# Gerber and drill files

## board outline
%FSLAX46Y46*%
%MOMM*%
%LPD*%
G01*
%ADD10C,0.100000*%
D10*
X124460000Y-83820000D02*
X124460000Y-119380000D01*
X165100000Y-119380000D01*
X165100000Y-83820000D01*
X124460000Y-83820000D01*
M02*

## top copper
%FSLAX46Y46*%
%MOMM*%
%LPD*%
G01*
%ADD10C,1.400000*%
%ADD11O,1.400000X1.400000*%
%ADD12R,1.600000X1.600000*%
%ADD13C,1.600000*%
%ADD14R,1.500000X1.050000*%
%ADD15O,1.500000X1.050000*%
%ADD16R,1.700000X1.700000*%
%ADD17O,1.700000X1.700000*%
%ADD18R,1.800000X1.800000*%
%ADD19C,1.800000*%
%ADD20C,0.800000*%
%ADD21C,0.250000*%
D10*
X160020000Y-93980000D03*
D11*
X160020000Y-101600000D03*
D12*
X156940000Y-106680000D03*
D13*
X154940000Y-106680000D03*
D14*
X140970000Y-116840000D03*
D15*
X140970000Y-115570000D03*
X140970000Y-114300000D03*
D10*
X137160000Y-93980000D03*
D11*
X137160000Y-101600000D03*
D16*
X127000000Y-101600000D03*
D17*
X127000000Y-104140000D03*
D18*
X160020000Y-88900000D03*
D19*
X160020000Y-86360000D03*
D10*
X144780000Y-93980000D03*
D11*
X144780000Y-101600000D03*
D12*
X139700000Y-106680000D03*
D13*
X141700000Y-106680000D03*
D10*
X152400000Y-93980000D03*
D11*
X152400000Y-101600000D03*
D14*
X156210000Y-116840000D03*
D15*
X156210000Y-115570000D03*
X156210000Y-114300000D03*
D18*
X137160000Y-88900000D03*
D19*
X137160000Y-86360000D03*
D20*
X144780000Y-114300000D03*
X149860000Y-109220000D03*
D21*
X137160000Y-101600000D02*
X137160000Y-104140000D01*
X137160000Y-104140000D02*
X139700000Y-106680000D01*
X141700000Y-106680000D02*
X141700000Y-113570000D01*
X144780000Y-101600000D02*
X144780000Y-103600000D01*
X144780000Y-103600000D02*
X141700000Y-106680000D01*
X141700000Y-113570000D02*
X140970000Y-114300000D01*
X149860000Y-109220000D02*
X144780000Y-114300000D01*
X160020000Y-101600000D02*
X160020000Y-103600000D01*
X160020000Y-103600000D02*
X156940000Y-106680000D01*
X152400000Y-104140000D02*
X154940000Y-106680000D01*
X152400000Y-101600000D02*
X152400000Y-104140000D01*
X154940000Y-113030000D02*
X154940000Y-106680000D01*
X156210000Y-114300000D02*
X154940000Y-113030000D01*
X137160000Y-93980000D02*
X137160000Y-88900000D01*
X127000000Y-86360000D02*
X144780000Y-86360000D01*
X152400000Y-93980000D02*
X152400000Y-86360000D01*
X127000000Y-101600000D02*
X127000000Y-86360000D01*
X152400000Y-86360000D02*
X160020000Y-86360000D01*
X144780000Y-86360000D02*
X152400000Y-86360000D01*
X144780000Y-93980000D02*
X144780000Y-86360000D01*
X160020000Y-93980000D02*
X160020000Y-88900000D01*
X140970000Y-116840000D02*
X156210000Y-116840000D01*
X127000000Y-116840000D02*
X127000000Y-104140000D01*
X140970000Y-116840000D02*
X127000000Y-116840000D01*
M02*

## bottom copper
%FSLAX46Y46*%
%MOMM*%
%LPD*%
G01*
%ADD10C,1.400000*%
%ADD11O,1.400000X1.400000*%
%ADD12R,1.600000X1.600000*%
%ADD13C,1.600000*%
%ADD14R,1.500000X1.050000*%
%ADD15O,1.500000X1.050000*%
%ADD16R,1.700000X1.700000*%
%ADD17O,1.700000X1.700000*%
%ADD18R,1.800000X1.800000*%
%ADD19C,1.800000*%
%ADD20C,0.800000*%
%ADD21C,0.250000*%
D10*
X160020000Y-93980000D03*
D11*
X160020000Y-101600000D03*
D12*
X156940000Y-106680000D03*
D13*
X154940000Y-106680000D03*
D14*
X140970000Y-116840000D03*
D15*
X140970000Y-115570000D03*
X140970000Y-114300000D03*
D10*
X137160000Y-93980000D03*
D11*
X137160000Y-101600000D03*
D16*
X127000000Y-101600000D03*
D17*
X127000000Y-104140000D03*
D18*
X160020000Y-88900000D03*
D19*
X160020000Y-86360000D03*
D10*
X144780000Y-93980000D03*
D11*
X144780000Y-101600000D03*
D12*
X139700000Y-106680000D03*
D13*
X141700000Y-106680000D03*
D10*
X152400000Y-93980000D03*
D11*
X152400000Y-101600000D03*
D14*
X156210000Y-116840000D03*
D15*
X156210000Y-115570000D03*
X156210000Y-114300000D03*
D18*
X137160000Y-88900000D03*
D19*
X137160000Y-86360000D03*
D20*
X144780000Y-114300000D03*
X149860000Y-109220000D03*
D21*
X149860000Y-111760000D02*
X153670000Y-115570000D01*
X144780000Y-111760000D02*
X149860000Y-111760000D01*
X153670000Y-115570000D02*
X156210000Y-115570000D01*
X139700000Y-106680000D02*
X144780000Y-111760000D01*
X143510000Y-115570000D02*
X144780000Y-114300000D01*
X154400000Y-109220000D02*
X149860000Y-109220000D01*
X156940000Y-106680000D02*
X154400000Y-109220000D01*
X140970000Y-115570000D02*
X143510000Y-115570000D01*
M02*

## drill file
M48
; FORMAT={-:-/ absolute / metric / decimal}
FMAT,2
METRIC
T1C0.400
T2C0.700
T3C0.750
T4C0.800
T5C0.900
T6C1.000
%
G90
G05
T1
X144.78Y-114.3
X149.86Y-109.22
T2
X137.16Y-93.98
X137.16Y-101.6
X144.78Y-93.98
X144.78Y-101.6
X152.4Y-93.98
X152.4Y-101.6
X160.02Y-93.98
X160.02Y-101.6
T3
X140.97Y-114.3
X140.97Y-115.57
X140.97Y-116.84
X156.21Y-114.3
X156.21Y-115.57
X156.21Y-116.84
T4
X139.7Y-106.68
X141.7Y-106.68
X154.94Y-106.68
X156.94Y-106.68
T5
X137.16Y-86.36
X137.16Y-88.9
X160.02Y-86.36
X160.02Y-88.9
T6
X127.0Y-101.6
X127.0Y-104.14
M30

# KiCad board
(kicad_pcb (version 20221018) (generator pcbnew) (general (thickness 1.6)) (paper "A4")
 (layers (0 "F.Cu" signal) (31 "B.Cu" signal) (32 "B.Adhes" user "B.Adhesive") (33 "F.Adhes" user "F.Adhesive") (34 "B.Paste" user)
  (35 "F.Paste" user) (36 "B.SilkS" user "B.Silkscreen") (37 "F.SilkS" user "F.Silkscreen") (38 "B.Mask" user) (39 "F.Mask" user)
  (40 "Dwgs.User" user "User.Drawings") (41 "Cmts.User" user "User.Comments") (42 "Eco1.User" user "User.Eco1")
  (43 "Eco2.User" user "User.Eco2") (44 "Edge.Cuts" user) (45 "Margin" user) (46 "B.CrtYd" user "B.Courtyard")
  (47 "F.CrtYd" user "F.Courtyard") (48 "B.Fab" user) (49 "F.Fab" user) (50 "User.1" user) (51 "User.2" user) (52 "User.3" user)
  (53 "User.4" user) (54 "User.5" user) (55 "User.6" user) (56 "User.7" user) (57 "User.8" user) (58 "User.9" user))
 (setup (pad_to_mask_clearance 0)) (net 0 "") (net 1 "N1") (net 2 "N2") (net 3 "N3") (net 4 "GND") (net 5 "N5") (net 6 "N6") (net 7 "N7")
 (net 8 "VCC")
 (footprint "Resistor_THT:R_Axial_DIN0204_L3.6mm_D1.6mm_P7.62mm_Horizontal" (layer "F.Cu") (at 160.02 93.98 -90)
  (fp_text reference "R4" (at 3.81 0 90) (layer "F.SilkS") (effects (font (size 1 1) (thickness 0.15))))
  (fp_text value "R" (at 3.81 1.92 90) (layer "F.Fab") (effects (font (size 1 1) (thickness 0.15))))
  (pad "1" thru_hole circle (at 0 0 270) (size 1.4 1.4) (drill 0.7) (layers "*.Cu" "*.Mask") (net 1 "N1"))
  (pad "2" thru_hole oval (at 7.62 0 270) (size 1.4 1.4) (drill 0.7) (layers "*.Cu" "*.Mask") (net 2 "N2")))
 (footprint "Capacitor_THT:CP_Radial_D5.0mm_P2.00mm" (layer "F.Cu") (at 156.94 106.68 180)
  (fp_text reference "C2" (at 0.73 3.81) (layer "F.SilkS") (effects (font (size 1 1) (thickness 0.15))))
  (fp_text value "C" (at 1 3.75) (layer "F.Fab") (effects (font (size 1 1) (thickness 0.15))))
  (pad "1" thru_hole rect (at 0 0 180) (size 1.6 1.6) (drill 0.8) (layers "*.Cu" "*.Mask") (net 2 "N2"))
  (pad "2" thru_hole circle (at 2 0 180) (size 1.6 1.6) (drill 0.8) (layers "*.Cu" "*.Mask") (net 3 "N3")))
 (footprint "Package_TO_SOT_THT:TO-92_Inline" (layer "F.Cu") (at 140.97 116.84 90)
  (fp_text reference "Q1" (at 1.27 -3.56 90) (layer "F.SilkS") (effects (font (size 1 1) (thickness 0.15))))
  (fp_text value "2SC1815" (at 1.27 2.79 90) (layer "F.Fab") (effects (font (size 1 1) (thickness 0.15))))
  (pad "1" thru_hole rect (at 0 0 90) (size 1.05 1.5) (drill 0.75) (layers "*.Cu" "*.Mask") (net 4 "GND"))
  (pad "2" thru_hole oval (at 1.27 0 90) (size 1.05 1.5) (drill 0.75) (layers "*.Cu" "*.Mask") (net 2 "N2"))
  (pad "3" thru_hole oval (at 2.54 0 90) (size 1.05 1.5) (drill 0.75) (layers "*.Cu" "*.Mask") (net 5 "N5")))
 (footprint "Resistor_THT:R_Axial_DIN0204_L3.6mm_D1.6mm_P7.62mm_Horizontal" (layer "F.Cu") (at 137.16 93.98 -90)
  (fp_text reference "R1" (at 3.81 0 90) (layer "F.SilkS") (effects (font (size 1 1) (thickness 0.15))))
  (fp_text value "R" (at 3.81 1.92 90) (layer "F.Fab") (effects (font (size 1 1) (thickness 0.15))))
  (pad "1" thru_hole circle (at 0 0 270) (size 1.4 1.4) (drill 0.7) (layers "*.Cu" "*.Mask") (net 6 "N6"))
  (pad "2" thru_hole oval (at 7.62 0 270) (size 1.4 1.4) (drill 0.7) (layers "*.Cu" "*.Mask") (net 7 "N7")))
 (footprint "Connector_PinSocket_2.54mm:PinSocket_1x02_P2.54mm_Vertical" (layer "F.Cu") (at 127 101.6)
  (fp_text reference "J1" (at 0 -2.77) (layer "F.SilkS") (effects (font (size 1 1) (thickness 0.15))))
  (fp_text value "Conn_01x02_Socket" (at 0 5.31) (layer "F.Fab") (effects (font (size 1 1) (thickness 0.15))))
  (pad "1" thru_hole rect (at 0 0) (size 1.7 1.7) (drill 1) (layers "*.Cu" "*.Mask") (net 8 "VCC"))
  (pad "2" thru_hole oval (at 0 2.54) (size 1.7 1.7) (drill 1) (layers "*.Cu" "*.Mask") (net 4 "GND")))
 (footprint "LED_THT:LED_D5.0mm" (layer "F.Cu") (at 160.02 88.9 90)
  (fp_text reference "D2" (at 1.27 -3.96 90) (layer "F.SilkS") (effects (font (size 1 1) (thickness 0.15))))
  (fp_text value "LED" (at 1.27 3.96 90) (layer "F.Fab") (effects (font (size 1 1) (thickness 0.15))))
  (pad "1" thru_hole rect (at 0 0 90) (size 1.8 1.8) (drill 0.9) (layers "*.Cu" "*.Mask") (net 1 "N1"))
  (pad "2" thru_hole circle (at 2.54 0 90) (size 1.8 1.8) (drill 0.9) (layers "*.Cu" "*.Mask") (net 8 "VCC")))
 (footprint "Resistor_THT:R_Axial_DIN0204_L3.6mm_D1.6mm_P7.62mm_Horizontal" (layer "F.Cu") (at 144.78 93.98 -90)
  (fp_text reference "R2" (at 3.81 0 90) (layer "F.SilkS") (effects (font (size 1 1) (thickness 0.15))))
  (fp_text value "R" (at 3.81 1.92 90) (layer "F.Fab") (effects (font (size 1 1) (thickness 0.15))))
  (pad "1" thru_hole circle (at 0 0 270) (size 1.4 1.4) (drill 0.7) (layers "*.Cu" "*.Mask") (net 8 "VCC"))
  (pad "2" thru_hole oval (at 7.62 0 270) (size 1.4 1.4) (drill 0.7) (layers "*.Cu" "*.Mask") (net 5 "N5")))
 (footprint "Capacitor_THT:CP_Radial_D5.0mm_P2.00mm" (layer "F.Cu") (at 139.7 106.68)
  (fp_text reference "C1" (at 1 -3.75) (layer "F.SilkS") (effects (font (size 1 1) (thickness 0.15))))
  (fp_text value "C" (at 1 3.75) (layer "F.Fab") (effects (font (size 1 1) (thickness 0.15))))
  (pad "1" thru_hole rect (at 0 0) (size 1.6 1.6) (drill 0.8) (layers "*.Cu" "*.Mask") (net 7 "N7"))
  (pad "2" thru_hole circle (at 2 0) (size 1.6 1.6) (drill 0.8) (layers "*.Cu" "*.Mask") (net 5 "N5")))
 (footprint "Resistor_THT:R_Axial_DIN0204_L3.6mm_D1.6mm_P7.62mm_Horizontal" (layer "F.Cu") (at 152.4 93.98 -90)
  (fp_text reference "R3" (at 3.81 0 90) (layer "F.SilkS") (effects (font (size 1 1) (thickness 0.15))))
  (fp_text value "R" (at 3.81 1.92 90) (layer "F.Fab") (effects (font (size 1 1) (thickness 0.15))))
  (pad "1" thru_hole circle (at 0 0 270) (size 1.4 1.4) (drill 0.7) (layers "*.Cu" "*.Mask") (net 8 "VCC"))
  (pad "2" thru_hole oval (at 7.62 0 270) (size 1.4 1.4) (drill 0.7) (layers "*.Cu" "*.Mask") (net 3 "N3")))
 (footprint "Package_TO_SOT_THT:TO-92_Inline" (layer "F.Cu") (at 156.21 116.84 90)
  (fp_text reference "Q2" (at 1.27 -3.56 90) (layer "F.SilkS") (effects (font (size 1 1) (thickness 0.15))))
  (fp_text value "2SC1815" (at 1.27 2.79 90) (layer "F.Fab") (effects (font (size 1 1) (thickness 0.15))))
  (pad "1" thru_hole rect (at 0 0 90) (size 1.05 1.5) (drill 0.75) (layers "*.Cu" "*.Mask") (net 4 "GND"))
  (pad "2" thru_hole oval (at 1.27 0 90) (size 1.05 1.5) (drill 0.75) (layers "*.Cu" "*.Mask") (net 7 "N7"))
  (pad "3" thru_hole oval (at 2.54 0 90) (size 1.05 1.5) (drill 0.75) (layers "*.Cu" "*.Mask") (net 3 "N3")))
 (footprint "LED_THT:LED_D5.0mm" (layer "F.Cu") (at 137.16 88.9 90)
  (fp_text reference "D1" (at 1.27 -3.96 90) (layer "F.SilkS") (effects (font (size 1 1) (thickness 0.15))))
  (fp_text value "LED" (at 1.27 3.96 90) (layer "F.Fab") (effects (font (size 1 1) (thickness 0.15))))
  (pad "1" thru_hole rect (at 0 0 90) (size 1.8 1.8) (drill 0.9) (layers "*.Cu" "*.Mask") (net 6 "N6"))
  (pad "2" thru_hole circle (at 2.54 0 90) (size 1.8 1.8) (drill 0.9) (layers "*.Cu" "*.Mask") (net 8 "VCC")))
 (gr_poly
  (pts (xy 124.46 83.82) (xy 124.46 119.38) (xy 165.1 119.38) (xy 165.1 83.82)) (stroke (width 0.1) (type solid)) (fill none)
  (layer "Edge.Cuts"))
 (segment (start 137.16 101.6) (end 137.16 104.14) (width 0.25) (layer "F.Cu") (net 7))
 (segment (start 137.16 104.14) (end 139.7 106.68) (width 0.25) (layer "F.Cu") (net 7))
 (segment (start 149.86 111.76) (end 153.67 115.57) (width 0.25) (layer "B.Cu") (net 7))
 (segment (start 144.78 111.76) (end 149.86 111.76) (width 0.25) (layer "B.Cu") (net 7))
 (segment (start 153.67 115.57) (end 156.21 115.57) (width 0.25) (layer "B.Cu") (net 7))
 (segment (start 139.7 106.68) (end 144.78 111.76) (width 0.25) (layer "B.Cu") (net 7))
 (segment (start 141.7 106.68) (end 141.7 113.57) (width 0.25) (layer "F.Cu") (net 5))
 (segment (start 144.78 101.6) (end 144.78 103.6) (width 0.25) (layer "F.Cu") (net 5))
 (segment (start 144.78 103.6) (end 141.7 106.68) (width 0.25) (layer "F.Cu") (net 5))
 (segment (start 141.7 113.57) (end 140.97 114.3) (width 0.25) (layer "F.Cu") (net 5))
 (segment (start 149.86 109.22) (end 144.78 114.3) (width 0.25) (layer "F.Cu") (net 2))
 (segment (start 160.02 101.6) (end 160.02 103.6) (width 0.25) (layer "F.Cu") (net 2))
 (segment (start 160.02 103.6) (end 156.94 106.68) (width 0.25) (layer "F.Cu") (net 2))
 (via (at 144.78 114.3) (size 0.8) (drill 0.4) (layers "F.Cu" "B.Cu") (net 2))
 (via (at 149.86 109.22) (size 0.8) (drill 0.4) (layers "F.Cu" "B.Cu") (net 2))
 (segment (start 143.51 115.57) (end 144.78 114.3) (width 0.25) (layer "B.Cu") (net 2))
 (segment (start 154.4 109.22) (end 149.86 109.22) (width 0.25) (layer "B.Cu") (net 2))
 (segment (start 156.94 106.68) (end 154.4 109.22) (width 0.25) (layer "B.Cu") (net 2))
 (segment (start 140.97 115.57) (end 143.51 115.57) (width 0.25) (layer "B.Cu") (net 2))
 (segment (start 152.4 104.14) (end 154.94 106.68) (width 0.25) (layer "F.Cu") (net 3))
 (segment (start 152.4 101.6) (end 152.4 104.14) (width 0.25) (layer "F.Cu") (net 3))
 (segment (start 154.94 113.03) (end 154.94 106.68) (width 0.25) (layer "F.Cu") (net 3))
 (segment (start 156.21 114.3) (end 154.94 113.03) (width 0.25) (layer "F.Cu") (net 3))
 (segment (start 137.16 93.98) (end 137.16 88.9) (width 0.25) (layer "F.Cu") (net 6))
 (segment (start 127 86.36) (end 144.78 86.36) (width 0.25) (layer "F.Cu") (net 8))
 (segment (start 152.4 93.98) (end 152.4 86.36) (width 0.25) (layer "F.Cu") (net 8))
 (segment (start 127 101.6) (end 127 86.36) (width 0.25) (layer "F.Cu") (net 8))
 (segment (start 152.4 86.36) (end 160.02 86.36) (width 0.25) (layer "F.Cu") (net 8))
 (segment (start 144.78 86.36) (end 152.4 86.36) (width 0.25) (layer "F.Cu") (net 8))
 (segment (start 144.78 93.98) (end 144.78 86.36) (width 0.25) (layer "F.Cu") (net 8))
 (segment (start 160.02 93.98) (end 160.02 88.9) (width 0.25) (layer "F.Cu") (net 1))
 (segment (start 140.97 116.84) (end 156.21 116.84) (width 0.25) (layer "F.Cu") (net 4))
 (segment (start 127 116.84) (end 127 104.14) (width 0.25) (layer "F.Cu") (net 4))
 (segment (start 140.97 116.84) (end 127 116.84) (width 0.25) (layer "F.Cu") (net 4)))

